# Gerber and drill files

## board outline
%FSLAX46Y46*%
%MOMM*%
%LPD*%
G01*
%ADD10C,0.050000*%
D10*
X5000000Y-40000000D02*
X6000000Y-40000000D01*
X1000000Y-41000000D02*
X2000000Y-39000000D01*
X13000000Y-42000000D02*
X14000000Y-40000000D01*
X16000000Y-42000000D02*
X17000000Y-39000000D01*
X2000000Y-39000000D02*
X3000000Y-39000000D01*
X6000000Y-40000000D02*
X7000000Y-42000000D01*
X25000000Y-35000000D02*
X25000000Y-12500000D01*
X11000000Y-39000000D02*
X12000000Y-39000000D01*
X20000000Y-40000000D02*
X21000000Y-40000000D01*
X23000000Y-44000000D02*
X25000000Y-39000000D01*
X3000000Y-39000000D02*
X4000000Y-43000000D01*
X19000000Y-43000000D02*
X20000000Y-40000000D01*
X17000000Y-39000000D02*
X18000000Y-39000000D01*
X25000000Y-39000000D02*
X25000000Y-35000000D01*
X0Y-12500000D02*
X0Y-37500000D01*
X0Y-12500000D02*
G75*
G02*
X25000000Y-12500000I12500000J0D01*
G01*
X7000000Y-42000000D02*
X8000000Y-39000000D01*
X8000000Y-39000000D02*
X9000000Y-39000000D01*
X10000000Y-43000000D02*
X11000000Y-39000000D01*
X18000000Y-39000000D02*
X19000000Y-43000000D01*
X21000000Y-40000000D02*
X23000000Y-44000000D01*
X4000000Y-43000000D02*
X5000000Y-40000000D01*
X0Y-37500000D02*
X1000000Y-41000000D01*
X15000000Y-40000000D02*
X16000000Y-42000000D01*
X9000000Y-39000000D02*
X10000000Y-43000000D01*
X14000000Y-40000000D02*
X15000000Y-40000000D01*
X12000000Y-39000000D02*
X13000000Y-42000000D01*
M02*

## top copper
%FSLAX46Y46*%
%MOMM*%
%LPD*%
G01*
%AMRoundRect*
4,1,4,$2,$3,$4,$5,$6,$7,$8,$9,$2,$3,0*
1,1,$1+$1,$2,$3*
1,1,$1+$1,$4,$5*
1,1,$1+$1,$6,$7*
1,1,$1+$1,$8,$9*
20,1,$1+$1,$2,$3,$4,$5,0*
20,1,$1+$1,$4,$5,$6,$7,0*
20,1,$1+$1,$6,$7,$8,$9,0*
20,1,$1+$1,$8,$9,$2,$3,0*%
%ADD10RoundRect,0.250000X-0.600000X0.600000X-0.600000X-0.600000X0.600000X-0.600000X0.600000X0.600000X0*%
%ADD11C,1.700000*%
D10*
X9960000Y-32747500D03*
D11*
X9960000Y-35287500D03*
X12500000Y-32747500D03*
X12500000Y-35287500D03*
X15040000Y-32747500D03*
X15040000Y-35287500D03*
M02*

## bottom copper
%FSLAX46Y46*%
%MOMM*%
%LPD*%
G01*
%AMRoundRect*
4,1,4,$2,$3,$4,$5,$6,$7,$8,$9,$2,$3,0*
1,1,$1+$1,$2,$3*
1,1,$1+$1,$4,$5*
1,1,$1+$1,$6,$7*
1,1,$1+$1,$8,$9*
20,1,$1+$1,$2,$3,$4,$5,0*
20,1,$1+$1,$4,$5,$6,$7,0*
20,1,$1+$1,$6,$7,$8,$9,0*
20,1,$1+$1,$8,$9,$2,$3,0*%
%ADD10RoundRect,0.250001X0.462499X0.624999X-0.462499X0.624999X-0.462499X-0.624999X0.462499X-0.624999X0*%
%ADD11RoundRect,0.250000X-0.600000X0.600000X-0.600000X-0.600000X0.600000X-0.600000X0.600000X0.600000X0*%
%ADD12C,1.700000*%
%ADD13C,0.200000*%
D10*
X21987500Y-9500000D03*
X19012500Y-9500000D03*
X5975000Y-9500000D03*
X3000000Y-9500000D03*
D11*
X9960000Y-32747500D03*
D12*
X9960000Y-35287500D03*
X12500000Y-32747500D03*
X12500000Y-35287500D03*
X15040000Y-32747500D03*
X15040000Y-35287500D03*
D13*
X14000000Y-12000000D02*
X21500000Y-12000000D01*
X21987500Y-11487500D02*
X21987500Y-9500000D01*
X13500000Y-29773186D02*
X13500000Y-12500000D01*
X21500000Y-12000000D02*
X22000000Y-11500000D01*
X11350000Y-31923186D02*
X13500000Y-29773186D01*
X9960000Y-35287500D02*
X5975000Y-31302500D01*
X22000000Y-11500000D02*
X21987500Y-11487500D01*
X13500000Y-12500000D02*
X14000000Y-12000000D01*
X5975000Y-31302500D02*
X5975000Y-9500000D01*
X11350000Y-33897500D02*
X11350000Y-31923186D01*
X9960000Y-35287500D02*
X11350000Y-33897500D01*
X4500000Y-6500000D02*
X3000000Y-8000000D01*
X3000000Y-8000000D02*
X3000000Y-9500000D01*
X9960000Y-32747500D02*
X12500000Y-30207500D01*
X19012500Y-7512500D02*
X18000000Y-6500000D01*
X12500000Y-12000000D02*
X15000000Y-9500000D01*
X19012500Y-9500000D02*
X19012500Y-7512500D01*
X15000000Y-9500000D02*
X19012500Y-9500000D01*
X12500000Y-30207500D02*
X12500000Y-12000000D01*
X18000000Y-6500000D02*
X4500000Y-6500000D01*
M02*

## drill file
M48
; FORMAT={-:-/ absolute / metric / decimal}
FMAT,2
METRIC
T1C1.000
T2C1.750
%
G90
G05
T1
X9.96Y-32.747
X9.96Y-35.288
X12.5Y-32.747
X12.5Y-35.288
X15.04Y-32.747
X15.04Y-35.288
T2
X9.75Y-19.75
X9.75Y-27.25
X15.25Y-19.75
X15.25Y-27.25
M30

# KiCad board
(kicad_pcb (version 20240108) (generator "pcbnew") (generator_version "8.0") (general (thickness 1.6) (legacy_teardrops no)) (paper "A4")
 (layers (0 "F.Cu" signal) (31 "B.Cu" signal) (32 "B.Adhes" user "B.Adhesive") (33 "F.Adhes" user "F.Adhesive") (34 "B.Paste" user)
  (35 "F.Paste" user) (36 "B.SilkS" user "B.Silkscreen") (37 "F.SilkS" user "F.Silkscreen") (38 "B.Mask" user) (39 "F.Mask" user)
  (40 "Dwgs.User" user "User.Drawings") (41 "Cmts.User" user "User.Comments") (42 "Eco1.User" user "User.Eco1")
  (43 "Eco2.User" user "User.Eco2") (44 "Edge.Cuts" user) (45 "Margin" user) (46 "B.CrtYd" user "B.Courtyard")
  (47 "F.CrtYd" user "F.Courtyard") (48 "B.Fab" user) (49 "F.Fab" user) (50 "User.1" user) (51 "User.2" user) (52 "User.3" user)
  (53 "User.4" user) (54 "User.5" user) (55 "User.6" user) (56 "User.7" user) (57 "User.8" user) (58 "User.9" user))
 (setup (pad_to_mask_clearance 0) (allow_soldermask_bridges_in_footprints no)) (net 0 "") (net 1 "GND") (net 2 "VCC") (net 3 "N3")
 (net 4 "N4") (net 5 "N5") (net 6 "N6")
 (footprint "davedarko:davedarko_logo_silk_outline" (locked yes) (layer "F.Cu") (at 20 33)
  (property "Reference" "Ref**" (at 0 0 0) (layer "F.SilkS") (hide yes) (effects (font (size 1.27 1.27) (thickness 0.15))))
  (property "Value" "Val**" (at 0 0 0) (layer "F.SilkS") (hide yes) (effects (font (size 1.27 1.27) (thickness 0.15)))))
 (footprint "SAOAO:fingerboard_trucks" (layer "F.Cu") (at 12.5 23.5)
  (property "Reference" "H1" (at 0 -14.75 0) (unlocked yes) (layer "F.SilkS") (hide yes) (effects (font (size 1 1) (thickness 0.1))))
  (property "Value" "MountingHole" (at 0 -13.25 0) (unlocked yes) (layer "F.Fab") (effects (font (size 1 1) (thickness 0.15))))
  (pad "" np_thru_hole circle (at -2.75 -3.75) (size 1.75 1.75) (drill 1.75) (layers "F&B.Cu" "*.Mask"))
  (pad "" np_thru_hole circle (at -2.75 3.75) (size 1.75 1.75) (drill 1.75) (layers "F&B.Cu" "*.Mask"))
  (pad "" np_thru_hole circle (at 2.75 -3.75) (size 1.75 1.75) (drill 1.75) (layers "F&B.Cu" "*.Mask"))
  (pad "" np_thru_hole circle (at 2.75 3.75) (size 1.75 1.75) (drill 1.75) (layers "F&B.Cu" "*.Mask")))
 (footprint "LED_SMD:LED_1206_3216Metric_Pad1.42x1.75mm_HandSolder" (layer "B.Cu") (at 20.5 9.5 180)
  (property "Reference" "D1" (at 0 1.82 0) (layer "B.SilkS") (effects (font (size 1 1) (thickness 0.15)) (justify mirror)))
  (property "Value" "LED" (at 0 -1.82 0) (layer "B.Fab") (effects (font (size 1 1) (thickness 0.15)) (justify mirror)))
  (pad "1" smd roundrect (at -1.4875 0 180) (size 1.425 1.75) (layers "B.Cu" "B.Paste" "B.Mask") (roundrect_rratio 0.175439) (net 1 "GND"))
  (pad "2" smd roundrect (at 1.4875 0 180) (size 1.425 1.75) (layers "B.Cu" "B.Paste" "B.Mask") (roundrect_rratio 0.175439) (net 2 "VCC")))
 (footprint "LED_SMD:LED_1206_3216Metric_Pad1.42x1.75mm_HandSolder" (layer "B.Cu") (at 4.4875 9.5 180)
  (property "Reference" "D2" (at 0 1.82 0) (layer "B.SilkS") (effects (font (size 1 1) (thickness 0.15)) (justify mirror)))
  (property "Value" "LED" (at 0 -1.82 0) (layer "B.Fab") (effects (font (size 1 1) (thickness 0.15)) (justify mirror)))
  (pad "1" smd roundrect (at -1.4875 0 180) (size 1.425 1.75) (layers "B.Cu" "B.Paste" "B.Mask") (roundrect_rratio 0.175439) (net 1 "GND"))
  (pad "2" smd roundrect (at 1.4875 0 180) (size 1.425 1.75) (layers "B.Cu" "B.Paste" "B.Mask") (roundrect_rratio 0.175439) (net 2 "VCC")))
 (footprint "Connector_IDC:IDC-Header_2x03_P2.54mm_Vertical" (layer "B.Cu") (at 9.96 32.7475 -90)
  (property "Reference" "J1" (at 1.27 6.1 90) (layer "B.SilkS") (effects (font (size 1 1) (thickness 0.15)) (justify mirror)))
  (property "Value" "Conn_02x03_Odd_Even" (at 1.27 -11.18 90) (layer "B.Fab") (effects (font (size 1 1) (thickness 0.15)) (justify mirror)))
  (pad "1" thru_hole roundrect (at 0 0 270) (size 1.7 1.7) (drill 1) (layers "*.Cu" "*.Mask") (remove_unused_layers no)
   (roundrect_rratio 0.147059) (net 2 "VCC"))
  (pad "2" thru_hole circle (at 2.54 0 270) (size 1.7 1.7) (drill 1) (layers "*.Cu" "*.Mask") (remove_unused_layers no) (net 1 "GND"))
  (pad "3" thru_hole circle (at 0 -2.54 270) (size 1.7 1.7) (drill 1) (layers "*.Cu" "*.Mask") (remove_unused_layers no) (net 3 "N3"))
  (pad "4" thru_hole circle (at 2.54 -2.54 270) (size 1.7 1.7) (drill 1) (layers "*.Cu" "*.Mask") (remove_unused_layers no) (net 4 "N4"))
  (pad "5" thru_hole circle (at 0 -5.08 270) (size 1.7 1.7) (drill 1) (layers "*.Cu" "*.Mask") (remove_unused_layers no) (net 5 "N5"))
  (pad "6" thru_hole circle (at 2.54 -5.08 270) (size 1.7 1.7) (drill 1) (layers "*.Cu" "*.Mask") (remove_unused_layers no) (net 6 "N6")))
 (gr_line (start 5 40) (end 6 40) (stroke (width 0.05) (type default)) (layer "Edge.Cuts"))
 (gr_line (start 1 41) (end 2 39) (stroke (width 0.05) (type default)) (layer "Edge.Cuts"))
 (gr_line (start 13 42) (end 14 40) (stroke (width 0.05) (type default)) (layer "Edge.Cuts"))
 (gr_line (start 16 42) (end 17 39) (stroke (width 0.05) (type default)) (layer "Edge.Cuts"))
 (gr_line (start 2 39) (end 3 39) (stroke (width 0.05) (type default)) (layer "Edge.Cuts"))
 (gr_line (start 6 40) (end 7 42) (stroke (width 0.05) (type default)) (layer "Edge.Cuts"))
 (gr_line (start 25 35) (end 25 12.5) (stroke (width 0.05) (type default)) (layer "Edge.Cuts"))
 (gr_line (start 11 39) (end 12 39) (stroke (width 0.05) (type default)) (layer "Edge.Cuts"))
 (gr_line (start 20 40) (end 21 40) (stroke (width 0.05) (type default)) (layer "Edge.Cuts"))
 (gr_line (start 23 44) (end 25 39) (stroke (width 0.05) (type default)) (layer "Edge.Cuts"))
 (gr_line (start 3 39) (end 4 43) (stroke (width 0.05) (type default)) (layer "Edge.Cuts"))
 (gr_line (start 19 43) (end 20 40) (stroke (width 0.05) (type default)) (layer "Edge.Cuts"))
 (gr_line (start 17 39) (end 18 39) (stroke (width 0.05) (type default)) (layer "Edge.Cuts"))
 (gr_line (start 25 39) (end 25 35) (stroke (width 0.05) (type default)) (layer "Edge.Cuts"))
 (gr_line (start 0 12.5) (end 0 37.5) (stroke (width 0.05) (type default)) (layer "Edge.Cuts"))
 (gr_arc (start 0 12.5) (mid 12.5 0) (end 25 12.5) (stroke (width 0.05) (type default)) (layer "Edge.Cuts"))
 (gr_line (start 7 42) (end 8 39) (stroke (width 0.05) (type default)) (layer "Edge.Cuts"))
 (gr_line (start 8 39) (end 9 39) (stroke (width 0.05) (type default)) (layer "Edge.Cuts"))
 (gr_line (start 10 43) (end 11 39) (stroke (width 0.05) (type default)) (layer "Edge.Cuts"))
 (gr_line (start 18 39) (end 19 43) (stroke (width 0.05) (type default)) (layer "Edge.Cuts"))
 (gr_line (start 21 40) (end 23 44) (stroke (width 0.05) (type default)) (layer "Edge.Cuts"))
 (gr_line (start 4 43) (end 5 40) (stroke (width 0.05) (type default)) (layer "Edge.Cuts"))
 (gr_line (start 0 37.5) (end 1 41) (stroke (width 0.05) (type default)) (layer "Edge.Cuts"))
 (gr_line (start 15 40) (end 16 42) (stroke (width 0.05) (type default)) (layer "Edge.Cuts"))
 (gr_line (start 9 39) (end 10 43) (stroke (width 0.05) (type default)) (layer "Edge.Cuts"))
 (gr_line (start 14 40) (end 15 40) (stroke (width 0.05) (type default)) (layer "Edge.Cuts"))
 (gr_line (start 12 39) (end 13 42) (stroke (width 0.05) (type default)) (layer "Edge.Cuts"))
 (segment (start 14 12) (end 21.5 12) (width 0.2) (layer "B.Cu") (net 1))
 (segment (start 21.9875 11.4875) (end 21.9875 9.5) (width 0.2) (layer "B.Cu") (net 1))
 (segment (start 13.5 29.773186) (end 13.5 12.5) (width 0.2) (layer "B.Cu") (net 1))
 (segment (start 21.5 12) (end 22 11.5) (width 0.2) (layer "B.Cu") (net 1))
 (segment (start 11.35 31.923186) (end 13.5 29.773186) (width 0.2) (layer "B.Cu") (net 1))
 (segment (start 9.96 35.2875) (end 5.975 31.3025) (width 0.2) (layer "B.Cu") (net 1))
 (segment (start 22 11.5) (end 21.9875 11.4875) (width 0.2) (layer "B.Cu") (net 1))
 (segment (start 13.5 12.5) (end 14 12) (width 0.2) (layer "B.Cu") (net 1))
 (segment (start 5.975 31.3025) (end 5.975 9.5) (width 0.2) (layer "B.Cu") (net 1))
 (segment (start 11.35 33.8975) (end 11.35 31.923186) (width 0.2) (layer "B.Cu") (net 1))
 (segment (start 9.96 35.2875) (end 11.35 33.8975) (width 0.2) (layer "B.Cu") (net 1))
 (segment (start 4.5 6.5) (end 3 8) (width 0.2) (layer "B.Cu") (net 2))
 (segment (start 3 8) (end 3 9.5) (width 0.2) (layer "B.Cu") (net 2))
 (segment (start 9.96 32.7475) (end 12.5 30.2075) (width 0.2) (layer "B.Cu") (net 2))
 (segment (start 19.0125 7.5125) (end 18 6.5) (width 0.2) (layer "B.Cu") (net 2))
 (segment (start 12.5 12) (end 15 9.5) (width 0.2) (layer "B.Cu") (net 2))
 (segment (start 19.0125 9.5) (end 19.0125 7.5125) (width 0.2) (layer "B.Cu") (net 2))
 (segment (start 15 9.5) (end 19.0125 9.5) (width 0.2) (layer "B.Cu") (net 2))
 (segment (start 12.5 30.2075) (end 12.5 12) (width 0.2) (layer "B.Cu") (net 2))
 (segment (start 18 6.5) (end 4.5 6.5) (width 0.2) (layer "B.Cu") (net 2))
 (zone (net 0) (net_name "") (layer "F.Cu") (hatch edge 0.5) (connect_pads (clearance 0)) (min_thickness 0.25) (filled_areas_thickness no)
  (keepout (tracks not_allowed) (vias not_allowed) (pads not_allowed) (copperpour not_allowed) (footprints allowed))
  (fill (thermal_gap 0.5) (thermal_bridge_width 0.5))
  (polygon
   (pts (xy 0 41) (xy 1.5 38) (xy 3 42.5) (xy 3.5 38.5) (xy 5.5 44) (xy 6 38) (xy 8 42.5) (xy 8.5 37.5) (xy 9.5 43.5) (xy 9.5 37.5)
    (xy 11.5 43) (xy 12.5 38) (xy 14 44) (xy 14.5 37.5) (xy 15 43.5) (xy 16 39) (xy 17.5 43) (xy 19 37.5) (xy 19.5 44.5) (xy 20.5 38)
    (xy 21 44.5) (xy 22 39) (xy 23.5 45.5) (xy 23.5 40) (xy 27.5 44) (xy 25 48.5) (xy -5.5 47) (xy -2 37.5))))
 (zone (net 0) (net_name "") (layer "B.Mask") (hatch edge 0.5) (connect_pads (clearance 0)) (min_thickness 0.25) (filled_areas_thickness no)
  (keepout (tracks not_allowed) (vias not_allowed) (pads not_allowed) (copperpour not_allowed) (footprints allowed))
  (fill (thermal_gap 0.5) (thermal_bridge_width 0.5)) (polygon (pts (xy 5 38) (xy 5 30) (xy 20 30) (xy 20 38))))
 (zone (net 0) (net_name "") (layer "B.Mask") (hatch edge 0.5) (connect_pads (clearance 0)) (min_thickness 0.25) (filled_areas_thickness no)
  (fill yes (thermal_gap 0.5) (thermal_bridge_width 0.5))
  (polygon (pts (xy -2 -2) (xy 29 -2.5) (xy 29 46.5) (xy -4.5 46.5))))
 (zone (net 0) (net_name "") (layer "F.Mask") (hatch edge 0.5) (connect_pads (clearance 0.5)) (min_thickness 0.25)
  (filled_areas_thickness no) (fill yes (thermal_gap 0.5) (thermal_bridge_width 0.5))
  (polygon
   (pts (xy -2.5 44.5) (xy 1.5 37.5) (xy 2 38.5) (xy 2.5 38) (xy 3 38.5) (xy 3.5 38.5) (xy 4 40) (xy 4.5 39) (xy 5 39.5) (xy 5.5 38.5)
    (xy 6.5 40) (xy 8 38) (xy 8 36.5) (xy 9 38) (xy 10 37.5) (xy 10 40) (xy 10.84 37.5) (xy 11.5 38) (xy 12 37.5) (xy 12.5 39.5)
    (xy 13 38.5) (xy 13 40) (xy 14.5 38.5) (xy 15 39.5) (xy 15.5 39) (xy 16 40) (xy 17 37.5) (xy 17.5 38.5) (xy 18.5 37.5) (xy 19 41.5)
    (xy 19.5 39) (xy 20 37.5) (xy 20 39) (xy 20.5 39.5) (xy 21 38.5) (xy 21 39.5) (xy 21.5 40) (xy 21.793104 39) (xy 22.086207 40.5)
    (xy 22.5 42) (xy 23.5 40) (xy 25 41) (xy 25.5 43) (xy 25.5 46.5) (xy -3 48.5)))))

